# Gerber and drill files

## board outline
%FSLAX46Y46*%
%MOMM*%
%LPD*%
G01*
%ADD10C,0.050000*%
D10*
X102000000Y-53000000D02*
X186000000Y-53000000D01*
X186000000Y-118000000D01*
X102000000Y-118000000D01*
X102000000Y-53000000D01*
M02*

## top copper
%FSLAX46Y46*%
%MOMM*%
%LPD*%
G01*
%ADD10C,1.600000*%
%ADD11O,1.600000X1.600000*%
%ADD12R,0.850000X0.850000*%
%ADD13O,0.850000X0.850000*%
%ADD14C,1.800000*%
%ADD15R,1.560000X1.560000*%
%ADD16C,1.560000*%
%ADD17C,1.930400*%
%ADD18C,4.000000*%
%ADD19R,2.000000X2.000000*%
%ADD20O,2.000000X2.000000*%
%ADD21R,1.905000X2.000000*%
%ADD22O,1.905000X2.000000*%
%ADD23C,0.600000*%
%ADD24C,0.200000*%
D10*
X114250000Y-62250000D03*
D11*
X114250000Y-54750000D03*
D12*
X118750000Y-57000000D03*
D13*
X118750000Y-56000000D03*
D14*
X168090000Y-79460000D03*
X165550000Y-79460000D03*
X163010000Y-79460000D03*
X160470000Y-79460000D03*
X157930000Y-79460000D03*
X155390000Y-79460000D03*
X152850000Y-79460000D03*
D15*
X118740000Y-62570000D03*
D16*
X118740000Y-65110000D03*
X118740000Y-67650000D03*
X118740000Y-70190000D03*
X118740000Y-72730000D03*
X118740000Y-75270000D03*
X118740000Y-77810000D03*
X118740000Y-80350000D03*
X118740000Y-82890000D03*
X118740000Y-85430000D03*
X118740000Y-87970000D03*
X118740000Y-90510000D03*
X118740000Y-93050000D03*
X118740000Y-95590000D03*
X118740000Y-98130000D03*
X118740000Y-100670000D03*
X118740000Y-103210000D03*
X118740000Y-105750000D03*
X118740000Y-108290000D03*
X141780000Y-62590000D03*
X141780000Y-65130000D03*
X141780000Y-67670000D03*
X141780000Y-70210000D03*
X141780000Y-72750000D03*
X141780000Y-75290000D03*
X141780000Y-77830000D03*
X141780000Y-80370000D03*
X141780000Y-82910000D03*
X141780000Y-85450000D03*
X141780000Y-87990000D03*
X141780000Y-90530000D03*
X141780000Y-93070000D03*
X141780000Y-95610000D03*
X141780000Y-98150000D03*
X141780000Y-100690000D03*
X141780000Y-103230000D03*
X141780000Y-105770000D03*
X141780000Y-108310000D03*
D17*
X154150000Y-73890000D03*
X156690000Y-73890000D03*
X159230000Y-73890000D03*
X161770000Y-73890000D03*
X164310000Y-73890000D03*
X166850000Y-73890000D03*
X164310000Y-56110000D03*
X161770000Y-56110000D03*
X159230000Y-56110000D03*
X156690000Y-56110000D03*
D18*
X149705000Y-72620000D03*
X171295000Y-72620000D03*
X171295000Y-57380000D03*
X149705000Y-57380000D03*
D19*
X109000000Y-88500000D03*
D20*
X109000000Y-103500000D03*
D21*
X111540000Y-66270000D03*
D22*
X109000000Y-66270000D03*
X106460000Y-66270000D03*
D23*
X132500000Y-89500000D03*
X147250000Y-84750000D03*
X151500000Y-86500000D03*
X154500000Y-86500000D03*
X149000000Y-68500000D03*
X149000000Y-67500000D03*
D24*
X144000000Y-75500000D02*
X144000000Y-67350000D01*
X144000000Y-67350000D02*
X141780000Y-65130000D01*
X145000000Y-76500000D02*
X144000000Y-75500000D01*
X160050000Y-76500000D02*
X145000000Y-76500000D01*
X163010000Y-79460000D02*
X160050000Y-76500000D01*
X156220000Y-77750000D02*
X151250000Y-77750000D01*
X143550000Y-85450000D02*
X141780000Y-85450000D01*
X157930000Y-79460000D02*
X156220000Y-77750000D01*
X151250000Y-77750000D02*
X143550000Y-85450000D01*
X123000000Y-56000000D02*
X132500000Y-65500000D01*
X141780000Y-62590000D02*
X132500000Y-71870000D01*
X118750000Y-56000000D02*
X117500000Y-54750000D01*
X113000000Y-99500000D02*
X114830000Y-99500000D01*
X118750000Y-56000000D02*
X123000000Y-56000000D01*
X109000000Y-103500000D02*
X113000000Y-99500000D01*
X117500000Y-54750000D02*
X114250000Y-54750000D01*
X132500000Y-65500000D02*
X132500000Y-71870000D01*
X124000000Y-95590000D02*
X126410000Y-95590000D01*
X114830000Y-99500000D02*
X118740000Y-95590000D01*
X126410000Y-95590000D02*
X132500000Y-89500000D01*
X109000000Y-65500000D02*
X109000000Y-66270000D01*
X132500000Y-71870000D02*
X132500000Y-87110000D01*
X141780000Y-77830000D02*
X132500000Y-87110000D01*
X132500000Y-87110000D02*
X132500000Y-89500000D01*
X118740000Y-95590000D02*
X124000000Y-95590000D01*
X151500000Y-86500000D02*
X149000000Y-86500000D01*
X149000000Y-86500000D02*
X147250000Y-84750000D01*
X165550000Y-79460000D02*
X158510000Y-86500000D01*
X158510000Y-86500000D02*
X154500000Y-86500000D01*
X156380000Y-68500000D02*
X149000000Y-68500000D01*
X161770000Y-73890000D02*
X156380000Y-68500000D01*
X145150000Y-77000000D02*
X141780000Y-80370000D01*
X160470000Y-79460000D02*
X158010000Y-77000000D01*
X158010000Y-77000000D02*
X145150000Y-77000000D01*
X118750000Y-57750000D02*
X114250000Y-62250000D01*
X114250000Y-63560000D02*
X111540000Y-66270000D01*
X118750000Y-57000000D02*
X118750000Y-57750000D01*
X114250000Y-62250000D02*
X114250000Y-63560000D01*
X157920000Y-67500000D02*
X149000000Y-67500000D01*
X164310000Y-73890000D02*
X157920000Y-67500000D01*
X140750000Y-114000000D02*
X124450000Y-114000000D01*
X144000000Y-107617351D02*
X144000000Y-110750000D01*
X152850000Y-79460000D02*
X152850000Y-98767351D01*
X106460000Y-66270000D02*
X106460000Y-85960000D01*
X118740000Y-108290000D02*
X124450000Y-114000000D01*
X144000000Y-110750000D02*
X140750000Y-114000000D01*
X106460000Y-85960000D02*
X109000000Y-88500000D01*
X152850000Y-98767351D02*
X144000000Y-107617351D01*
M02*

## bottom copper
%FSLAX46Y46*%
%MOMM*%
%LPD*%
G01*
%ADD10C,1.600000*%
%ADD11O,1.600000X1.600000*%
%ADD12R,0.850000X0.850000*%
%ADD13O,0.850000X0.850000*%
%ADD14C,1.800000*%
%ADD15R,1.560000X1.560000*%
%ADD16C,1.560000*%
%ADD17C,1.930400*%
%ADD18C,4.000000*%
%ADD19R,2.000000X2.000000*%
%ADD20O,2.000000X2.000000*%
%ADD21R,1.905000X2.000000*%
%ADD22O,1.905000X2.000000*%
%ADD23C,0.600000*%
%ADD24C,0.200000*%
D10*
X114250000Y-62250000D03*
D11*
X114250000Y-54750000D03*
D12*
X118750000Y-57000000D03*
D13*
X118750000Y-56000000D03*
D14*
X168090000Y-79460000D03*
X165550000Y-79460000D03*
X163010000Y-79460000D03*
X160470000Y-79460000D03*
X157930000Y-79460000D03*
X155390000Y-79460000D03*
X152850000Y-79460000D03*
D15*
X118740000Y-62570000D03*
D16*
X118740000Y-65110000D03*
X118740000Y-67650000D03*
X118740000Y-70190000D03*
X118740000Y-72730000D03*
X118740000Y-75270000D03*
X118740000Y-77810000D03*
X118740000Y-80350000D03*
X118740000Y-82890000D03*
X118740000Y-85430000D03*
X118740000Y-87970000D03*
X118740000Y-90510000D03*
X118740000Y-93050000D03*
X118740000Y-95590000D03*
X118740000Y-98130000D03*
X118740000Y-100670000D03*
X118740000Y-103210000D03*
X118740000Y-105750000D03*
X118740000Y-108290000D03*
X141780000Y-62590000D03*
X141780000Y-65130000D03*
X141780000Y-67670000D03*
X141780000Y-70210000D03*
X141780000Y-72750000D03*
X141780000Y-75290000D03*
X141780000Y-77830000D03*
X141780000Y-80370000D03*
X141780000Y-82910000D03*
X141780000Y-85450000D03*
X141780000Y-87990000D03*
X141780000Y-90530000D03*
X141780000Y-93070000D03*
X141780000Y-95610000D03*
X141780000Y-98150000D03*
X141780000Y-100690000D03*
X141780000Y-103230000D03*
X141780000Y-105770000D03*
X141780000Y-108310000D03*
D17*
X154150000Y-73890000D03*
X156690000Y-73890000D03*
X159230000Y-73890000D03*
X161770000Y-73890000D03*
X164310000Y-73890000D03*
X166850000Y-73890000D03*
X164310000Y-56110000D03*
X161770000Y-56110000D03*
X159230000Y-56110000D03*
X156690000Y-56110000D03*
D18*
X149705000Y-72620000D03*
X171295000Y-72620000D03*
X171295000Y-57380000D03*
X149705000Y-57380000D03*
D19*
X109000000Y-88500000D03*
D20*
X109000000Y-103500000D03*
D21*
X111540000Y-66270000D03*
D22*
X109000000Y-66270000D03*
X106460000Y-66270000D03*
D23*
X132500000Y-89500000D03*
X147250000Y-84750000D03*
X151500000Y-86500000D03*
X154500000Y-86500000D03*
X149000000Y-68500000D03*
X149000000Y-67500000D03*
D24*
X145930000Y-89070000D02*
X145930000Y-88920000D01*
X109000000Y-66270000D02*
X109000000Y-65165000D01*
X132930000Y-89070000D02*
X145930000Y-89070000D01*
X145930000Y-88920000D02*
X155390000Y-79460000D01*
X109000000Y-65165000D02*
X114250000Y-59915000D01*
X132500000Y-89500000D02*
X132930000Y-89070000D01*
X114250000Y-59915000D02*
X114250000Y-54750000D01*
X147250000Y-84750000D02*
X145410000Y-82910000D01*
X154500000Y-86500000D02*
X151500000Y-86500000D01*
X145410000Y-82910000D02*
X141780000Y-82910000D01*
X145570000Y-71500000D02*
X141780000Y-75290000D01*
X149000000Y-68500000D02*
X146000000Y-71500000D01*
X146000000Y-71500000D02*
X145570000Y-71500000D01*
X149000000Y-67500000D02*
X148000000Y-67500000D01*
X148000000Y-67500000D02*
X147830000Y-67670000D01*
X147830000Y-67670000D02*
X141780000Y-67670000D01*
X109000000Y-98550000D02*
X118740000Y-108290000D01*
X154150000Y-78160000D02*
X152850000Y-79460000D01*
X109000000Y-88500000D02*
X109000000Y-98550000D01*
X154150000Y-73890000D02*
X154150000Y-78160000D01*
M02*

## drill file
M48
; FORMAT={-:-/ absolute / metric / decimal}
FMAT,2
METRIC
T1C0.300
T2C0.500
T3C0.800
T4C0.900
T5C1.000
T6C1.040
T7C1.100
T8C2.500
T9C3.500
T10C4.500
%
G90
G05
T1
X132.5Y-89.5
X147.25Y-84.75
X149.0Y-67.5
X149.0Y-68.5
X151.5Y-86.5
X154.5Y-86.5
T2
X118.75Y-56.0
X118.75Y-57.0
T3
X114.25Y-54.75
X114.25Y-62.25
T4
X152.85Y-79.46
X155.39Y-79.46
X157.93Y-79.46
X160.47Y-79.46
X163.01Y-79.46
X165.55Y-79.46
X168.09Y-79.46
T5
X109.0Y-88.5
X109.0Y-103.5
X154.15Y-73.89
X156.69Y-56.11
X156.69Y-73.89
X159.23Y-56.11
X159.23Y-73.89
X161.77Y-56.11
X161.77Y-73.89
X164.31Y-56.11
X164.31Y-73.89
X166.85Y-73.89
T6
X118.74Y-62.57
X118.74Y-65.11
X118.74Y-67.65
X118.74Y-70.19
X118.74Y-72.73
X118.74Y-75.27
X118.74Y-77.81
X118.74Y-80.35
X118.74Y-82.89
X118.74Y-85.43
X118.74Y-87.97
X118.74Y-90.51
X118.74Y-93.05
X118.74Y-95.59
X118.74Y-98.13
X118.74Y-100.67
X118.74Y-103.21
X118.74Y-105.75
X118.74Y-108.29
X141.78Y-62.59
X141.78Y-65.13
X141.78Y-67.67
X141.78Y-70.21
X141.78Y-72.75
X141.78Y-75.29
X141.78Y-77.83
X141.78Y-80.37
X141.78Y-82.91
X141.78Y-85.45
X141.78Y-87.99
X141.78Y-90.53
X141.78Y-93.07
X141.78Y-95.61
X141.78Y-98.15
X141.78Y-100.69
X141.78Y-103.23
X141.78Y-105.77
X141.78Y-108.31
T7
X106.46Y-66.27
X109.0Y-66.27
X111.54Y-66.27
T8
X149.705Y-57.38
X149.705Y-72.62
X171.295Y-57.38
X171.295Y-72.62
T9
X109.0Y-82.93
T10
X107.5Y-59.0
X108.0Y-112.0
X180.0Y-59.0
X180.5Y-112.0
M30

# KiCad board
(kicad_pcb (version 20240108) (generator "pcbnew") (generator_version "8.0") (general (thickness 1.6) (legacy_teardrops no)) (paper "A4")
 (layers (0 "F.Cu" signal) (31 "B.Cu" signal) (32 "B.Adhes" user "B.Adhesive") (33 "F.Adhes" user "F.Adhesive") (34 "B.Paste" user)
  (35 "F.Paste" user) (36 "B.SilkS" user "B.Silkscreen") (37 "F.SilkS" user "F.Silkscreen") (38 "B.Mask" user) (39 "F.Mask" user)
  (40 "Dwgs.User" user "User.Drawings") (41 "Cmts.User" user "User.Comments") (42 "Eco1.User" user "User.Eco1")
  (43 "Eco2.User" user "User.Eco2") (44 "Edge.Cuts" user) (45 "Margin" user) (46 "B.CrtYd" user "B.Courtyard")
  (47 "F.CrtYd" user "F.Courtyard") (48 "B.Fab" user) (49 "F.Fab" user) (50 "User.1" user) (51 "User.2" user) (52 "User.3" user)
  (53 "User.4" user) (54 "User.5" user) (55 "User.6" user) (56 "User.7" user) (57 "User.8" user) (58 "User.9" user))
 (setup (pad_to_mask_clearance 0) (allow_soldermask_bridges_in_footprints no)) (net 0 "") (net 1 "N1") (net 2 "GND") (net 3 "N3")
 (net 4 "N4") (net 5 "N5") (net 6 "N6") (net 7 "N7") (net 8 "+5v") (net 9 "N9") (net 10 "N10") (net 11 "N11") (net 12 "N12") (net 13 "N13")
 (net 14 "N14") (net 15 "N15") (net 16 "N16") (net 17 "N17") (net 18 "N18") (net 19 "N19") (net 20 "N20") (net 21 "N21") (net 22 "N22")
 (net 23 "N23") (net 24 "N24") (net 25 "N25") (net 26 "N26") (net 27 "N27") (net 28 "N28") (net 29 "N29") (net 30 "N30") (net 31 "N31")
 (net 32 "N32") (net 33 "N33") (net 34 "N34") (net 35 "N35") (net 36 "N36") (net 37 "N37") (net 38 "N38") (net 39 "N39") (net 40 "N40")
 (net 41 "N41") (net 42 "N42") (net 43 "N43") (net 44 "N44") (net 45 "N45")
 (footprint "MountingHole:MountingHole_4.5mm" (layer "F.Cu") (at 107.5 59)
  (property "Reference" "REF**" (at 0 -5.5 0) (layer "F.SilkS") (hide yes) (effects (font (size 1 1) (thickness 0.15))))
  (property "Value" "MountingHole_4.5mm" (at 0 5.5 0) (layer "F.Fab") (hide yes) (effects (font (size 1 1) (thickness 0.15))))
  (pad "" np_thru_hole circle (at 0 0) (size 4.5 4.5) (drill 4.5) (layers "*.Cu" "*.Mask")))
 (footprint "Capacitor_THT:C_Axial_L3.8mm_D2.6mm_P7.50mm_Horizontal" (layer "F.Cu") (at 114.25 62.25 90)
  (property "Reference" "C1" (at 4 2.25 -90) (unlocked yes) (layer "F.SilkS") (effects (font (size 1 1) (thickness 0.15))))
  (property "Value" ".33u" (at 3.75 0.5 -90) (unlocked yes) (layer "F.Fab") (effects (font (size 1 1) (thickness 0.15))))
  (pad "1" thru_hole circle (at 0 0 90) (size 1.6 1.6) (drill 0.8) (layers "*.Cu" "*.Mask") (remove_unused_layers no) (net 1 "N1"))
  (pad "2" thru_hole oval (at 7.5 0 90) (size 1.6 1.6) (drill 0.8) (layers "*.Cu" "*.Mask") (remove_unused_layers no) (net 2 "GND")))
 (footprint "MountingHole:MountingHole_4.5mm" (layer "F.Cu") (at 180.5 112)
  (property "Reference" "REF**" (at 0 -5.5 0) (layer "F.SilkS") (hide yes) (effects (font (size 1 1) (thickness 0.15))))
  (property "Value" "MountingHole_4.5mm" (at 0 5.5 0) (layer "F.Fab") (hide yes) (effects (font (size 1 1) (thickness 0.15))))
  (pad "" np_thru_hole circle (at 0 0) (size 4.5 4.5) (drill 4.5) (layers "*.Cu" "*.Mask")))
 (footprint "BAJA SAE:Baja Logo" (layer "F.Cu") (at 181.25 79.5 -90)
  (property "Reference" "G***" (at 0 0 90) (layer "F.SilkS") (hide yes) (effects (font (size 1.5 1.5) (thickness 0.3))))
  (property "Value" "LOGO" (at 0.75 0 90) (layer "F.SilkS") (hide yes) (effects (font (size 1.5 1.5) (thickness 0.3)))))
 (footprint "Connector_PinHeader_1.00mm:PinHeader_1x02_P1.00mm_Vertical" (layer "F.Cu") (at 118.75 57 180)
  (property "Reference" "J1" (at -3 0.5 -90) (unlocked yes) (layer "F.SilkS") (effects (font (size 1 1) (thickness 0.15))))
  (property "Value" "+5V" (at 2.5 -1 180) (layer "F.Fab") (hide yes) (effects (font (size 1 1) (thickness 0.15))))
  (pad "1" thru_hole rect (at 0 0 180) (size 0.85 0.85) (drill 0.5) (layers "*.Cu" "*.Mask") (remove_unused_layers no) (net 1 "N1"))
  (pad "2" thru_hole oval (at 0 1 180) (size 0.85 0.85) (drill 0.5) (layers "*.Cu" "*.Mask") (remove_unused_layers no) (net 2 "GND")))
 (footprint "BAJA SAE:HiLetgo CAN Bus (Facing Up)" (layer "F.Cu") (at 160.5 97.5 -90)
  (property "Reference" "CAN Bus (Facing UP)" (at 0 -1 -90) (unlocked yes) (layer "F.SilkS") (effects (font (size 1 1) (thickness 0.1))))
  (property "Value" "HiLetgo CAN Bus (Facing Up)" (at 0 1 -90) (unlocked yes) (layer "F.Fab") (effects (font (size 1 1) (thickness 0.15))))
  (pad "1" thru_hole circle (at -18.04 -7.59 270) (size 1.8 1.8) (drill 0.9) (layers "*.Cu" "*.Mask") (remove_unused_layers no) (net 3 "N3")
   (solder_mask_margin 0.102))
  (pad "2" thru_hole circle (at -18.04 -5.05 270) (size 1.8 1.8) (drill 0.9) (layers "*.Cu" "*.Mask") (remove_unused_layers no) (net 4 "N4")
   (solder_mask_margin 0.102))
  (pad "3" thru_hole circle (at -18.04 -2.51 270) (size 1.8 1.8) (drill 0.9) (layers "*.Cu" "*.Mask") (remove_unused_layers no) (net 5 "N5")
   (solder_mask_margin 0.102))
  (pad "4" thru_hole circle (at -18.04 0.03 270) (size 1.8 1.8) (drill 0.9) (layers "*.Cu" "*.Mask") (remove_unused_layers no) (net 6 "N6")
   (solder_mask_margin 0.102))
  (pad "5" thru_hole circle (at -18.04 2.57 270) (size 1.8 1.8) (drill 0.9) (layers "*.Cu" "*.Mask") (remove_unused_layers no) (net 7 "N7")
   (solder_mask_margin 0.102))
  (pad "6" thru_hole circle (at -18.04 5.11 270) (size 1.8 1.8) (drill 0.9) (layers "*.Cu" "*.Mask") (remove_unused_layers no) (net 2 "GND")
   (solder_mask_margin 0.102))
  (pad "7" thru_hole circle (at -18.04 7.65 270) (size 1.8 1.8) (drill 0.9) (layers "*.Cu" "*.Mask") (remove_unused_layers no) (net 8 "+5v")
   (solder_mask_margin 0.102)))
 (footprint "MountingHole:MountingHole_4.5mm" (layer "F.Cu") (at 180 59)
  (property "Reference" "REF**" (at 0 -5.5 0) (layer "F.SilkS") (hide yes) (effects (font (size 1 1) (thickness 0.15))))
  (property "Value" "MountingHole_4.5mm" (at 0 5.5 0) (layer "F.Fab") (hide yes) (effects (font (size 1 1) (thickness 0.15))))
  (pad "" np_thru_hole circle (at 0 0) (size 4.5 4.5) (drill 4.5) (layers "*.Cu" "*.Mask")))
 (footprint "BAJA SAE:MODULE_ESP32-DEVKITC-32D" (layer "F.Cu") (at 130.5 81.5)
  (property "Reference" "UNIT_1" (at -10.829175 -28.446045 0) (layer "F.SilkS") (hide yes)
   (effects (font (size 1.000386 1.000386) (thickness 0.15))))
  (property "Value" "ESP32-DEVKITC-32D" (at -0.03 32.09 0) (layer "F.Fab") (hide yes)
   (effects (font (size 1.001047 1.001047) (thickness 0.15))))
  (pad "J2-1" thru_hole rect (at -11.76 -18.93) (size 1.56 1.56) (drill 1.04) (layers "*.Cu" "*.Mask") (remove_unused_layers no)
   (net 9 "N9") (solder_mask_margin 0.102))
  (pad "J2-2" thru_hole circle (at -11.76 -16.39) (size 1.56 1.56) (drill 1.04) (layers "*.Cu" "*.Mask") (remove_unused_layers no)
   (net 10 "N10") (solder_mask_margin 0.102))
  (pad "J2-3" thru_hole circle (at -11.76 -13.85) (size 1.56 1.56) (drill 1.04) (layers "*.Cu" "*.Mask") (remove_unused_layers no)
   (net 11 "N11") (solder_mask_margin 0.102))
  (pad "J2-4" thru_hole circle (at -11.76 -11.31) (size 1.56 1.56) (drill 1.04) (layers "*.Cu" "*.Mask") (remove_unused_layers no)
   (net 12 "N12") (solder_mask_margin 0.102))
  (pad "J2-5" thru_hole circle (at -11.76 -8.77) (size 1.56 1.56) (drill 1.04) (layers "*.Cu" "*.Mask") (remove_unused_layers no)
   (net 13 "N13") (solder_mask_margin 0.102))
  (pad "J2-6" thru_hole circle (at -11.76 -6.23) (size 1.56 1.56) (drill 1.04) (layers "*.Cu" "*.Mask") (remove_unused_layers no)
   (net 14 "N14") (solder_mask_margin 0.102))
  (pad "J2-7" thru_hole circle (at -11.76 -3.69) (size 1.56 1.56) (drill 1.04) (layers "*.Cu" "*.Mask") (remove_unused_layers no)
   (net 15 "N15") (solder_mask_margin 0.102))
  (pad "J2-8" thru_hole circle (at -11.76 -1.15) (size 1.56 1.56) (drill 1.04) (layers "*.Cu" "*.Mask") (remove_unused_layers no)
   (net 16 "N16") (solder_mask_margin 0.102))
  (pad "J2-9" thru_hole circle (at -11.76 1.39) (size 1.56 1.56) (drill 1.04) (layers "*.Cu" "*.Mask") (remove_unused_layers no)
   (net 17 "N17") (solder_mask_margin 0.102))
  (pad "J2-10" thru_hole circle (at -11.76 3.93) (size 1.56 1.56) (drill 1.04) (layers "*.Cu" "*.Mask") (remove_unused_layers no)
   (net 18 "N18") (solder_mask_margin 0.102))
  (pad "J2-11" thru_hole circle (at -11.76 6.47) (size 1.56 1.56) (drill 1.04) (layers "*.Cu" "*.Mask") (remove_unused_layers no)
   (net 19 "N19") (solder_mask_margin 0.102))
  (pad "J2-12" thru_hole circle (at -11.76 9.01) (size 1.56 1.56) (drill 1.04) (layers "*.Cu" "*.Mask") (remove_unused_layers no)
   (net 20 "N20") (solder_mask_margin 0.102))
  (pad "J2-13" thru_hole circle (at -11.76 11.55) (size 1.56 1.56) (drill 1.04) (layers "*.Cu" "*.Mask") (remove_unused_layers no)
   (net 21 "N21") (solder_mask_margin 0.102))
  (pad "J2-14" thru_hole circle (at -11.76 14.09) (size 1.56 1.56) (drill 1.04) (layers "*.Cu" "*.Mask") (remove_unused_layers no)
   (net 2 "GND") (solder_mask_margin 0.102))
  (pad "J2-15" thru_hole circle (at -11.76 16.63) (size 1.56 1.56) (drill 1.04) (layers "*.Cu" "*.Mask") (remove_unused_layers no)
   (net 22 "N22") (solder_mask_margin 0.102))
  (pad "J2-16" thru_hole circle (at -11.76 19.17) (size 1.56 1.56) (drill 1.04) (layers "*.Cu" "*.Mask") (remove_unused_layers no)
   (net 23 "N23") (solder_mask_margin 0.102))
  (pad "J2-17" thru_hole circle (at -11.76 21.71) (size 1.56 1.56) (drill 1.04) (layers "*.Cu" "*.Mask") (remove_unused_layers no)
   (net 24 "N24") (solder_mask_margin 0.102))
  (pad "J2-18" thru_hole circle (at -11.76 24.25) (size 1.56 1.56) (drill 1.04) (layers "*.Cu" "*.Mask") (remove_unused_layers no)
   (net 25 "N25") (solder_mask_margin 0.102))
  (pad "J2-19" thru_hole circle (at -11.76 26.79) (size 1.56 1.56) (drill 1.04) (layers "*.Cu" "*.Mask") (remove_unused_layers no)
   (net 8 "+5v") (solder_mask_margin 0.102))
  (pad "J3-1" thru_hole circle (at 11.28 -18.91) (size 1.56 1.56) (drill 1.04) (layers "*.Cu" "*.Mask") (remove_unused_layers no)
   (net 2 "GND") (solder_mask_margin 0.102))
  (pad "J3-2" thru_hole circle (at 11.28 -16.37) (size 1.56 1.56) (drill 1.04) (layers "*.Cu" "*.Mask") (remove_unused_layers no)
   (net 5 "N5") (solder_mask_margin 0.102))
  (pad "J3-3" thru_hole circle (at 11.28 -13.83) (size 1.56 1.56) (drill 1.04) (layers "*.Cu" "*.Mask") (remove_unused_layers no)
   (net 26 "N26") (solder_mask_margin 0.102))
  (pad "J3-4" thru_hole circle (at 11.28 -11.29) (size 1.56 1.56) (drill 1.04) (layers "*.Cu" "*.Mask") (remove_unused_layers no)
   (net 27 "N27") (solder_mask_margin 0.102))
  (pad "J3-5" thru_hole circle (at 11.28 -8.75) (size 1.56 1.56) (drill 1.04) (layers "*.Cu" "*.Mask") (remove_unused_layers no)
   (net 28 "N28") (solder_mask_margin 0.102))
  (pad "J3-6" thru_hole circle (at 11.28 -6.21) (size 1.56 1.56) (drill 1.04) (layers "*.Cu" "*.Mask") (remove_unused_layers no)
   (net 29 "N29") (solder_mask_margin 0.102))
  (pad "J3-7" thru_hole circle (at 11.28 -3.67) (size 1.56 1.56) (drill 1.04) (layers "*.Cu" "*.Mask") (remove_unused_layers no)
   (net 2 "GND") (solder_mask_margin 0.102))
  (pad "J3-8" thru_hole circle (at 11.28 -1.13) (size 1.56 1.56) (drill 1.04) (layers "*.Cu" "*.Mask") (remove_unused_layers no)
   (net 6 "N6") (solder_mask_margin 0.102))
  (pad "J3-9" thru_hole circle (at 11.28 1.41) (size 1.56 1.56) (drill 1.04) (layers "*.Cu" "*.Mask") (remove_unused_layers no) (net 4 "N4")
   (solder_mask_margin 0.102))
  (pad "J3-10" thru_hole circle (at 11.28 3.95) (size 1.56 1.56) (drill 1.04) (layers "*.Cu" "*.Mask") (remove_unused_layers no)
   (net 7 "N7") (solder_mask_margin 0.102))
  (pad "J3-11" thru_hole circle (at 11.28 6.49) (size 1.56 1.56) (drill 1.04) (layers "*.Cu" "*.Mask") (remove_unused_layers no)
   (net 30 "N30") (solder_mask_margin 0.102))
  (pad "J3-12" thru_hole circle (at 11.28 9.03) (size 1.56 1.56) (drill 1.04) (layers "*.Cu" "*.Mask") (remove_unused_layers no)
   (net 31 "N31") (solder_mask_margin 0.102))
  (pad "J3-13" thru_hole circle (at 11.28 11.57) (size 1.56 1.56) (drill 1.04) (layers "*.Cu" "*.Mask") (remove_unused_layers no)
   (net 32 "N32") (solder_mask_margin 0.102))
  (pad "J3-14" thru_hole circle (at 11.28 14.11) (size 1.56 1.56) (drill 1.04) (layers "*.Cu" "*.Mask") (remove_unused_layers no)
   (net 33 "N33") (solder_mask_margin 0.102))
  (pad "J3-15" thru_hole circle (at 11.28 16.65) (size 1.56 1.56) (drill 1.04) (layers "*.Cu" "*.Mask") (remove_unused_layers no)
   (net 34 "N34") (solder_mask_margin 0.102))
  (pad "J3-16" thru_hole circle (at 11.28 19.19) (size 1.56 1.56) (drill 1.04) (layers "*.Cu" "*.Mask") (remove_unused_layers no)
   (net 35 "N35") (solder_mask_margin 0.102))
  (pad "J3-17" thru_hole circle (at 11.28 21.73) (size 1.56 1.56) (drill 1.04) (layers "*.Cu" "*.Mask") (remove_unused_layers no)
   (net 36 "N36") (solder_mask_margin 0.102))
  (pad "J3-18" thru_hole circle (at 11.28 24.27) (size 1.56 1.56) (drill 1.04) (layers "*.Cu" "*.Mask") (remove_unused_layers no)
   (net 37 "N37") (solder_mask_margin 0.102))
  (pad "J3-19" thru_hole circle (at 11.28 26.81) (size 1.56 1.56) (drill 1.04) (layers "*.Cu" "*.Mask") (remove_unused_layers no)
   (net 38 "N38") (solder_mask_margin 0.102)))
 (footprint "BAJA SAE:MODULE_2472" (layer "F.Cu") (at 160.5 65)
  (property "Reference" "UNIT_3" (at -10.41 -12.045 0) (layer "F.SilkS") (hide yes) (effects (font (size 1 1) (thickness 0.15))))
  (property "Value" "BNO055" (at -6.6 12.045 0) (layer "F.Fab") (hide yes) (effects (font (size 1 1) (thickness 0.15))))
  (pad "1" thru_hole circle (at -6.35 8.89) (size 1.9304 1.9304) (drill 1) (layers "*.Cu" "*.Mask") (remove_unused_layers no) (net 8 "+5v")
   (solder_mask_margin 0.102))
  (pad "2" thru_hole circle (at -3.81 8.89) (size 1.9304 1.9304) (drill 1) (layers "*.Cu" "*.Mask") (remove_unused_layers no) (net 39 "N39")
   (solder_mask_margin 0.102))
  (pad "3" thru_hole circle (at -1.27 8.89) (size 1.9304 1.9304) (drill 1) (layers "*.Cu" "*.Mask") (remove_unused_layers no) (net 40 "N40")
   (solder_mask_margin 0.102))
  (pad "4" thru_hole circle (at 1.27 8.89) (size 1.9304 1.9304) (drill 1) (layers "*.Cu" "*.Mask") (remove_unused_layers no) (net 29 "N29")
   (solder_mask_margin 0.102))
  (pad "5" thru_hole circle (at 3.81 8.89) (size 1.9304 1.9304) (drill 1) (layers "*.Cu" "*.Mask") (remove_unused_layers no) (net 26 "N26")
   (solder_mask_margin 0.102))
  (pad "6" thru_hole circle (at 6.35 8.89) (size 1.9304 1.9304) (drill 1) (layers "*.Cu" "*.Mask") (remove_unused_layers no) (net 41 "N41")
   (solder_mask_margin 0.102))
  (pad "7" thru_hole circle (at 3.81 -8.89) (size 1.9304 1.9304) (drill 1) (layers "*.Cu" "*.Mask") (remove_unused_layers no) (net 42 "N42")
   (solder_mask_margin 0.102))
  (pad "8" thru_hole circle (at 1.27 -8.89) (size 1.9304 1.9304) (drill 1) (layers "*.Cu" "*.Mask") (remove_unused_layers no) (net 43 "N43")
   (solder_mask_margin 0.102))
  (pad "9" thru_hole circle (at -1.27 -8.89) (size 1.9304 1.9304) (drill 1) (layers "*.Cu" "*.Mask") (remove_unused_layers no)
   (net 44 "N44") (solder_mask_margin 0.102))
  (pad "10" thru_hole circle (at -3.81 -8.89) (size 1.9304 1.9304) (drill 1) (layers "*.Cu" "*.Mask") (remove_unused_layers no)
   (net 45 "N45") (solder_mask_margin 0.102))
  (pad "SH1" thru_hole circle (at -10.795 7.62) (size 4 4) (drill 2.5) (layers "*.Cu" "*.Mask") (remove_unused_layers no)
   (solder_mask_margin 0.102))
  (pad "SH2" thru_hole circle (at 10.795 7.62) (size 4 4) (drill 2.5) (layers "*.Cu" "*.Mask") (remove_unused_layers no)
   (solder_mask_margin 0.102))
  (pad "SH3" thru_hole circle (at 10.795 -7.62) (size 4 4) (drill 2.5) (layers "*.Cu" "*.Mask") (remove_unused_layers no)
   (solder_mask_margin 0.102))
  (pad "SH4" thru_hole circle (at -10.795 -7.62) (size 4 4) (drill 2.5) (layers "*.Cu" "*.Mask") (remove_unused_layers no)
   (solder_mask_margin 0.102)))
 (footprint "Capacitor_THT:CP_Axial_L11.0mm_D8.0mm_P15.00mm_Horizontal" (layer "F.Cu") (at 109 88.5 -90)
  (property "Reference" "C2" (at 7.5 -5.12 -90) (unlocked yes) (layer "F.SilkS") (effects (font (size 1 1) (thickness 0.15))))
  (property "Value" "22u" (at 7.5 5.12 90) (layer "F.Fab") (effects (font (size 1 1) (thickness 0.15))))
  (pad "1" thru_hole rect (at 0 0 270) (size 2 2) (drill 1) (layers "*.Cu" "*.Mask") (remove_unused_layers no) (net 8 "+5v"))
  (pad "2" thru_hole oval (at 15 0 270) (size 2 2) (drill 1) (layers "*.Cu" "*.Mask") (remove_unused_layers no) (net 2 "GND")))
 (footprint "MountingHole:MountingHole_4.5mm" (layer "F.Cu") (at 108 112)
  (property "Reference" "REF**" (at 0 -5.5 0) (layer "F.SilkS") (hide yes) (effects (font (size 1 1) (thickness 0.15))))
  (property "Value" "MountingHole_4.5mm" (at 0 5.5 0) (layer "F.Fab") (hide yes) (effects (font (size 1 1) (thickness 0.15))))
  (pad "" np_thru_hole circle (at 0 0) (size 4.5 4.5) (drill 4.5) (layers "*.Cu" "*.Mask")))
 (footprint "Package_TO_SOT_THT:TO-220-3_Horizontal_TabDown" (layer "F.Cu") (at 111.54 66.27 180)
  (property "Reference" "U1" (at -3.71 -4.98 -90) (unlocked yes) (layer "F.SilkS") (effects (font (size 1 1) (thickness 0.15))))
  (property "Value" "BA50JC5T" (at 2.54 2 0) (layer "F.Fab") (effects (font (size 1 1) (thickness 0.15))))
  (pad "" np_thru_hole oval (at 2.54 -16.66 180) (size 3.5 3.5) (drill 3.5) (layers "*.Cu" "*.Mask"))
  (pad "1" thru_hole rect (at 0 0 180) (size 1.905 2) (drill 1.1) (layers "*.Cu" "*.Mask") (remove_unused_layers no) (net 1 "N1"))
  (pad "2" thru_hole oval (at 2.54 0 180) (size 1.905 2) (drill 1.1) (layers "*.Cu" "*.Mask") (remove_unused_layers no) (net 2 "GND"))
  (pad "3" thru_hole oval (at 5.08 0 180) (size 1.905 2) (drill 1.1) (layers "*.Cu" "*.Mask") (remove_unused_layers no) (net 8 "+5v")))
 (gr_rect (start 102 53) (end 186 118) (stroke (width 0.05) (type default)) (fill none) (layer "Edge.Cuts"))
 (segment (start 144 75.5) (end 144 67.35) (width 0.2) (layer "F.Cu") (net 5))
 (segment (start 144 67.35) (end 141.78 65.13) (width 0.2) (layer "F.Cu") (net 5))
 (segment (start 145 76.5) (end 144 75.5) (width 0.2) (layer "F.Cu") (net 5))
 (segment (start 160.05 76.5) (end 145 76.5) (width 0.2) (layer "F.Cu") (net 5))
 (segment (start 163.01 79.46) (end 160.05 76.5) (width 0.2) (layer "F.Cu") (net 5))
 (segment (start 156.22 77.75) (end 151.25 77.75) (width 0.2) (layer "F.Cu") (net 7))
 (segment (start 143.55 85.45) (end 141.78 85.45) (width 0.2) (layer "F.Cu") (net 7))
 (segment (start 157.93 79.46) (end 156.22 77.75) (width 0.2) (layer "F.Cu") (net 7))
 (segment (start 151.25 77.75) (end 143.55 85.45) (width 0.2) (layer "F.Cu") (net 7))
 (segment (start 123 56) (end 132.5 65.5) (width 0.2) (layer "F.Cu") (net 2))
 (segment (start 141.78 62.59) (end 132.5 71.87) (width 0.2) (layer "F.Cu") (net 2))
 (segment (start 118.75 56) (end 117.5 54.75) (width 0.2) (layer "F.Cu") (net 2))
 (segment (start 113 99.5) (end 114.83 99.5) (width 0.2) (layer "F.Cu") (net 2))
 (segment (start 118.75 56) (end 123 56) (width 0.2) (layer "F.Cu") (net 2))
 (segment (start 109 103.5) (end 113 99.5) (width 0.2) (layer "F.Cu") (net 2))
 (segment (start 117.5 54.75) (end 114.25 54.75) (width 0.2) (layer "F.Cu") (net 2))
 (segment (start 132.5 65.5) (end 132.5 71.87) (width 0.2) (layer "F.Cu") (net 2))
 (segment (start 124 95.59) (end 126.41 95.59) (width 0.2) (layer "F.Cu") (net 2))
 (segment (start 114.83 99.5) (end 118.74 95.59) (width 0.2) (layer "F.Cu") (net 2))
 (segment (start 126.41 95.59) (end 132.5 89.5) (width 0.2) (layer "F.Cu") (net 2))
 (segment (start 109 65.5) (end 109 66.27) (width 0.2) (layer "F.Cu") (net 2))
 (segment (start 132.5 71.87) (end 132.5 87.11) (width 0.2) (layer "F.Cu") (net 2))
 (segment (start 141.78 77.83) (end 132.5 87.11) (width 0.2) (layer "F.Cu") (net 2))
 (segment (start 132.5 87.11) (end 132.5 89.5) (width 0.2) (layer "F.Cu") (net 2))
 (segment (start 118.74 95.59) (end 124 95.59) (width 0.2) (layer "F.Cu") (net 2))
 (via (at 132.5 89.5) (size 0.6) (drill 0.3) (layers "F.Cu" "B.Cu") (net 2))
 (segment (start 145.93 89.07) (end 145.93 88.92) (width 0.2) (layer "B.Cu") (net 2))
 (segment (start 109 66.27) (end 109 65.165) (width 0.2) (layer "B.Cu") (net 2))
 (segment (start 132.93 89.07) (end 145.93 89.07) (width 0.2) (layer "B.Cu") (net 2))
 (segment (start 145.93 88.92) (end 155.39 79.46) (width 0.2) (layer "B.Cu") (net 2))
 (segment (start 109 65.165) (end 114.25 59.915) (width 0.2) (layer "B.Cu") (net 2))
 (segment (start 132.5 89.5) (end 132.93 89.07) (width 0.2) (layer "B.Cu") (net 2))
 (segment (start 114.25 59.915) (end 114.25 54.75) (width 0.2) (layer "B.Cu") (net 2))
 (segment (start 151.5 86.5) (end 149 86.5) (width 0.2) (layer "F.Cu") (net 4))
 (segment (start 149 86.5) (end 147.25 84.75) (width 0.2) (layer "F.Cu") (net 4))
 (segment (start 165.55 79.46) (end 158.51 86.5) (width 0.2) (layer "F.Cu") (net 4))
 (segment (start 158.51 86.5) (end 154.5 86.5) (width 0.2) (layer "F.Cu") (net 4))
 (via (at 147.25 84.75) (size 0.6) (drill 0.3) (layers "F.Cu" "B.Cu") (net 4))
 (via (at 151.5 86.5) (size 0.6) (drill 0.3) (layers "F.Cu" "B.Cu") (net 4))
 (via (at 154.5 86.5) (size 0.6) (drill 0.3) (layers "F.Cu" "B.Cu") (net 4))
 (segment (start 147.25 84.75) (end 145.41 82.91) (width 0.2) (layer "B.Cu") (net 4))
 (segment (start 154.5 86.5) (end 151.5 86.5) (width 0.2) (layer "B.Cu") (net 4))
 (segment (start 145.41 82.91) (end 141.78 82.91) (width 0.2) (layer "B.Cu") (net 4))
 (segment (start 156.38 68.5) (end 149 68.5) (width 0.2) (layer "F.Cu") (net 29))
 (segment (start 161.77 73.89) (end 156.38 68.5) (width 0.2) (layer "F.Cu") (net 29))
 (via (at 149 68.5) (size 0.6) (drill 0.3) (layers "F.Cu" "B.Cu") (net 29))
 (segment (start 145.57 71.5) (end 141.78 75.29) (width 0.2) (layer "B.Cu") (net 29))
 (segment (start 149 68.5) (end 146 71.5) (width 0.2) (layer "B.Cu") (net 29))
 (segment (start 146 71.5) (end 145.57 71.5) (width 0.2) (layer "B.Cu") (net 29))
 (segment (start 145.15 77) (end 141.78 80.37) (width 0.2) (layer "F.Cu") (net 6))
 (segment (start 160.47 79.46) (end 158.01 77) (width 0.2) (layer "F.Cu") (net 6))
 (segment (start 158.01 77) (end 145.15 77) (width 0.2) (layer "F.Cu") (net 6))
 (segment (start 118.75 57.75) (end 114.25 62.25) (width 0.2) (layer "F.Cu") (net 1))
 (segment (start 114.25 63.56) (end 111.54 66.27) (width 0.2) (layer "F.Cu") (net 1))
 (segment (start 118.75 57) (end 118.75 57.75) (width 0.2) (layer "F.Cu") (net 1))
 (segment (start 114.25 62.25) (end 114.25 63.56) (width 0.2) (layer "F.Cu") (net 1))
 (segment (start 157.92 67.5) (end 149 67.5) (width 0.2) (layer "F.Cu") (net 26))
 (segment (start 164.31 73.89) (end 157.92 67.5) (width 0.2) (layer "F.Cu") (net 26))
 (via (at 149 67.5) (size 0.6) (drill 0.3) (layers "F.Cu" "B.Cu") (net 26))
 (segment (start 149 67.5) (end 148 67.5) (width 0.2) (layer "B.Cu") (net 26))
 (segment (start 148 67.5) (end 147.83 67.67) (width 0.2) (layer "B.Cu") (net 26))
 (segment (start 147.83 67.67) (end 141.78 67.67) (width 0.2) (layer "B.Cu") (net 26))
 (segment (start 140.75 114) (end 124.45 114) (width 0.2) (layer "F.Cu") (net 8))
 (segment (start 144 107.617351) (end 144 110.75) (width 0.2) (layer "F.Cu") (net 8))
 (segment (start 152.85 79.46) (end 152.85 98.767351) (width 0.2) (layer "F.Cu") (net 8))
 (segment (start 106.46 66.27) (end 106.46 85.96) (width 0.2) (layer "F.Cu") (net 8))
 (segment (start 118.74 108.29) (end 124.45 114) (width 0.2) (layer "F.Cu") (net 8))
 (segment (start 144 110.75) (end 140.75 114) (width 0.2) (layer "F.Cu") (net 8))
 (segment (start 106.46 85.96) (end 109 88.5) (width 0.2) (layer "F.Cu") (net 8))
 (segment (start 152.85 98.767351) (end 144 107.617351) (width 0.2) (layer "F.Cu") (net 8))
 (segment (start 109 98.55) (end 118.74 108.29) (width 0.2) (layer "B.Cu") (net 8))
 (segment (start 154.15 78.16) (end 152.85 79.46) (width 0.2) (layer "B.Cu") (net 8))
 (segment (start 109 88.5) (end 109 98.55) (width 0.2) (layer "B.Cu") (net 8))
 (segment (start 154.15 73.89) (end 154.15 78.16) (width 0.2) (layer "B.Cu") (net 8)))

